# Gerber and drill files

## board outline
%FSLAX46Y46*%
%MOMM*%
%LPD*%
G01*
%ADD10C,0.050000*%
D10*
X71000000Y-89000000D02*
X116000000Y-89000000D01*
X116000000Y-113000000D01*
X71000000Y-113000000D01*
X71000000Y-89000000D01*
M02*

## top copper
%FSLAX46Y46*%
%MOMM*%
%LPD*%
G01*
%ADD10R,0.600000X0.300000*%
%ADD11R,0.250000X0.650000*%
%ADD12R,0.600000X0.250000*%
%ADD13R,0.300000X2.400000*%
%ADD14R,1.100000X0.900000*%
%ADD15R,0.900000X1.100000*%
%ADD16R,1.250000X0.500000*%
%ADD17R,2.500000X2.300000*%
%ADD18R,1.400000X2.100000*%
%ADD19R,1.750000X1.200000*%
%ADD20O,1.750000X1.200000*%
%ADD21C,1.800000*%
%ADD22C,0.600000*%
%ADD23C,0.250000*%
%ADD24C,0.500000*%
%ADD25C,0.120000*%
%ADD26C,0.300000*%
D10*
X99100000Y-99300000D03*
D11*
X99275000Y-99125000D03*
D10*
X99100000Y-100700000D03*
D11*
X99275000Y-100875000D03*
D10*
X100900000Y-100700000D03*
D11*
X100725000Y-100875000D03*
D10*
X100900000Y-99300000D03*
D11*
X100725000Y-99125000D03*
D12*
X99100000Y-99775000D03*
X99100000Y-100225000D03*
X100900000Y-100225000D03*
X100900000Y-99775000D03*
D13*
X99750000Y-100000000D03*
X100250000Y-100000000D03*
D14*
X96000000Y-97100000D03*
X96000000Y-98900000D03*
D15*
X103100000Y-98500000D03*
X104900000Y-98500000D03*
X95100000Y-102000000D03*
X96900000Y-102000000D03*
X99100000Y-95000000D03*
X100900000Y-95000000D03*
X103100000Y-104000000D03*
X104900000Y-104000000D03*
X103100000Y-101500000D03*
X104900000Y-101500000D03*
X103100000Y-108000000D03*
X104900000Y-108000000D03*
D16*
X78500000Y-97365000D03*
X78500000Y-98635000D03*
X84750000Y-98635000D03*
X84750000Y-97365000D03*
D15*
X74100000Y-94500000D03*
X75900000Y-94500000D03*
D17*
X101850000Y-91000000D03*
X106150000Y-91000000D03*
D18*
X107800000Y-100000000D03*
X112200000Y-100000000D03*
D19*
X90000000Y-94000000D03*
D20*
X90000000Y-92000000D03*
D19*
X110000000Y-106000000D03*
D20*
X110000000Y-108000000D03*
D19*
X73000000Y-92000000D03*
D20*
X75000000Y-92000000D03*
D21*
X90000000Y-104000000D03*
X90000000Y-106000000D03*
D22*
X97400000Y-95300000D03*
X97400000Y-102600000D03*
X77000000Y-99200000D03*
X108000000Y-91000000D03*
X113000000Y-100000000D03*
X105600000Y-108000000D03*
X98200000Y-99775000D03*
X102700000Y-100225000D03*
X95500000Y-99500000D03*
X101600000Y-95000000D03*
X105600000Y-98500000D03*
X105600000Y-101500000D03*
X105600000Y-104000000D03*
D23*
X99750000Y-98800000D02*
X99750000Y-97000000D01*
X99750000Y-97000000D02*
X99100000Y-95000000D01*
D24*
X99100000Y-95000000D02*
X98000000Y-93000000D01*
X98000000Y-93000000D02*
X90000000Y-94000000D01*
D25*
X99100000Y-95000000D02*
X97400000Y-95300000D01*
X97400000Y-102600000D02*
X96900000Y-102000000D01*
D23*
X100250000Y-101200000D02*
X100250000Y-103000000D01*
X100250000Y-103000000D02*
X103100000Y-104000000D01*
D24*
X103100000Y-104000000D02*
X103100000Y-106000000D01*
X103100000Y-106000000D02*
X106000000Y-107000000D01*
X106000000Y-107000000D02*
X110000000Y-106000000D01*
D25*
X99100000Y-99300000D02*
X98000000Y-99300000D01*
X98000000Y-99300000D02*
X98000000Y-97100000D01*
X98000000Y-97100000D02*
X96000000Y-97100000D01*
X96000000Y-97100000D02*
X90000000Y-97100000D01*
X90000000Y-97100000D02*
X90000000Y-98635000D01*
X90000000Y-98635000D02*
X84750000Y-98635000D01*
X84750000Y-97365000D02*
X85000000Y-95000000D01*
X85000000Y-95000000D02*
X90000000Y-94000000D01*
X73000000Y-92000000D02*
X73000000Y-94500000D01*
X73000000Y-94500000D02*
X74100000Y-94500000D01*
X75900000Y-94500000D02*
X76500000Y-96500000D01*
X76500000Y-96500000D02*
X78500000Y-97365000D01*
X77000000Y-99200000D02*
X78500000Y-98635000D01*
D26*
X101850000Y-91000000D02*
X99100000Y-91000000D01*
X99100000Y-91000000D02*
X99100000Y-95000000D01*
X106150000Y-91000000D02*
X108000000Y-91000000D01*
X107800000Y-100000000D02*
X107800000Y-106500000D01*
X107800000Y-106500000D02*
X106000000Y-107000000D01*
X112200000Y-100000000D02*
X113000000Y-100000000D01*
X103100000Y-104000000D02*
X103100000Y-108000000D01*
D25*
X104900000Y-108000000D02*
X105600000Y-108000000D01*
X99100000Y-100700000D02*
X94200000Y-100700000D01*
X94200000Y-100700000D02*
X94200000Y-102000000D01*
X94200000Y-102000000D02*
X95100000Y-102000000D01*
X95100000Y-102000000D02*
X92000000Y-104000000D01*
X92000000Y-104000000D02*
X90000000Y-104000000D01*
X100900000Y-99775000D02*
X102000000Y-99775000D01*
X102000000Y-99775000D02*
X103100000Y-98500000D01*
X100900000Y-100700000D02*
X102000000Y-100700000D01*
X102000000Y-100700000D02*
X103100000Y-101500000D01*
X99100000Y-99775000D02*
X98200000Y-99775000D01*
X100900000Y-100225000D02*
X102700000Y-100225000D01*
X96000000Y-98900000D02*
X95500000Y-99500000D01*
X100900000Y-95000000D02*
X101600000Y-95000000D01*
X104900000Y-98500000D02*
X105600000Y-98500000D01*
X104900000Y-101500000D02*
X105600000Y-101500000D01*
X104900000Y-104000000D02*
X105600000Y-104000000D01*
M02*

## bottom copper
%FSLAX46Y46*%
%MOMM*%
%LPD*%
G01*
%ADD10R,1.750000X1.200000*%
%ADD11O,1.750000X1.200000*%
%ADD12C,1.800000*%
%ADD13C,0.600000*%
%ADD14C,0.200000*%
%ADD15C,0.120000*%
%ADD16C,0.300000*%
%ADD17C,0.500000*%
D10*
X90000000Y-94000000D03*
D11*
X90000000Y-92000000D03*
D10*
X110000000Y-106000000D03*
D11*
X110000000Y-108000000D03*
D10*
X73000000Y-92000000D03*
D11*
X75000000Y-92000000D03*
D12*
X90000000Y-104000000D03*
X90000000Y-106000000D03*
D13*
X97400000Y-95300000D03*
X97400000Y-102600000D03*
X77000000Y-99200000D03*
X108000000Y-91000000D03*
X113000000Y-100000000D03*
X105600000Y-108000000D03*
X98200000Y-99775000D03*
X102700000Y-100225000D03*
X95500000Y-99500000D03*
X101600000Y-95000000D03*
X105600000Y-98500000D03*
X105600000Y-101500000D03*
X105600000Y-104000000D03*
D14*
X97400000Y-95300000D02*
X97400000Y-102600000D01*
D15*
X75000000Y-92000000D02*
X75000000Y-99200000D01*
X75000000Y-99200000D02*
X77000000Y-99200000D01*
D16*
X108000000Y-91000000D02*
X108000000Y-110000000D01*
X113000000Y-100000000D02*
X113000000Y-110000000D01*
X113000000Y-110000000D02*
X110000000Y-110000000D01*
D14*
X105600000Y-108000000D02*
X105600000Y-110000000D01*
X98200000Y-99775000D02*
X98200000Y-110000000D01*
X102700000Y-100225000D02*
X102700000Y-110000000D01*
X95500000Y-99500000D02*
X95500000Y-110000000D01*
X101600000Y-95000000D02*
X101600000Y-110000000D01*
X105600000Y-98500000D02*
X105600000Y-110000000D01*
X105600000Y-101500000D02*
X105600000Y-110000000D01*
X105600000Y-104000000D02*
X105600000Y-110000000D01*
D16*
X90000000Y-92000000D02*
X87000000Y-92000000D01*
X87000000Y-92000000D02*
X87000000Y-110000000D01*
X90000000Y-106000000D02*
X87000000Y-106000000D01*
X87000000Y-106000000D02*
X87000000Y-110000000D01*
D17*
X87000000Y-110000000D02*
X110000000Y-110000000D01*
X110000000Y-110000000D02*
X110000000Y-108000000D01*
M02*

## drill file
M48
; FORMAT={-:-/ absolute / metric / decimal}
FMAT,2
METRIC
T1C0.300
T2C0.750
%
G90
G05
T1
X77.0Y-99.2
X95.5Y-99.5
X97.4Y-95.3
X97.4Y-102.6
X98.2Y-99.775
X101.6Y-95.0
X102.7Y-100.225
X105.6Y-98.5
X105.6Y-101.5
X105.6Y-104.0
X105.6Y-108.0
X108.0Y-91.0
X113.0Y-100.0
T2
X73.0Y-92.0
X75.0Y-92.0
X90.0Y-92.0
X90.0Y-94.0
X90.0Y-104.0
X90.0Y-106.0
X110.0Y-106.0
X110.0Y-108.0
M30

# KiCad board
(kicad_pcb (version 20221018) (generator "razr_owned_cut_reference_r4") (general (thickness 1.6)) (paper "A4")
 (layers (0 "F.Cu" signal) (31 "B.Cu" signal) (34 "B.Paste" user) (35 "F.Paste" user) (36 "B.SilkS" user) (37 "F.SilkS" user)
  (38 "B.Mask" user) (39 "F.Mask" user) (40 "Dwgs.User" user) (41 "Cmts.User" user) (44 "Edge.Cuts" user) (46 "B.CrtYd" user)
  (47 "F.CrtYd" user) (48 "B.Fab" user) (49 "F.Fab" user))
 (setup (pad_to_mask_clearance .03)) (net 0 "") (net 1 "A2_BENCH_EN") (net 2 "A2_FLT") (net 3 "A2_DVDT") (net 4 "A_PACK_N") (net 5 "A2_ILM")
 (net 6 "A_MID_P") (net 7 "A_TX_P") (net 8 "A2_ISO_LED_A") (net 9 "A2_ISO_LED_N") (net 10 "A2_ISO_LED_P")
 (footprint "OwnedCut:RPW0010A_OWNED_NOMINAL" (layer "F.Cu") (at 100 100)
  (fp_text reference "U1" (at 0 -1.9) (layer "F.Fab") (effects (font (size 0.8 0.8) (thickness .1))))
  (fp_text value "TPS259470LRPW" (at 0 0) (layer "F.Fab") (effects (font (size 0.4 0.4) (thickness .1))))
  (pad "1" smd rect (at -0.9 -0.7) (size 0.6 0.3) (layers "F.Cu" "F.Paste" "F.Mask") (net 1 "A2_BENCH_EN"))
  (pad "1" smd rect (at -0.725 -0.875) (size 0.25 0.65) (layers "F.Cu" "F.Paste" "F.Mask") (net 1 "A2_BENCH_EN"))
  (pad "4" smd rect (at -0.9 0.7) (size 0.6 0.3) (layers "F.Cu" "F.Paste" "F.Mask") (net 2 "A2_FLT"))
  (pad "4" smd rect (at -0.725 0.875) (size 0.25 0.65) (layers "F.Cu" "F.Paste" "F.Mask") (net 2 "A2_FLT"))
  (pad "7" smd rect (at 0.9 0.7) (size 0.6 0.3) (layers "F.Cu" "F.Paste" "F.Mask") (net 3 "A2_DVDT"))
  (pad "7" smd rect (at 0.725 0.875) (size 0.25 0.65) (layers "F.Cu" "F.Paste" "F.Mask") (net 3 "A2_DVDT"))
  (pad "10" smd rect (at 0.9 -0.7) (size 0.6 0.3) (layers "F.Cu" "F.Paste" "F.Mask"))
  (pad "10" smd rect (at 0.725 -0.875) (size 0.25 0.65) (layers "F.Cu" "F.Paste" "F.Mask"))
  (pad "2" smd rect (at -0.9 -0.225) (size 0.6 0.25) (layers "F.Cu" "F.Paste" "F.Mask") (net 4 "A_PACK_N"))
  (pad "3" smd rect (at -0.9 0.225) (size 0.6 0.25) (layers "F.Cu" "F.Paste" "F.Mask"))
  (pad "8" smd rect (at 0.9 0.225) (size 0.6 0.25) (layers "F.Cu" "F.Paste" "F.Mask") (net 4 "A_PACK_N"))
  (pad "9" smd rect (at 0.9 -0.225) (size 0.6 0.25) (layers "F.Cu" "F.Paste" "F.Mask") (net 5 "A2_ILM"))
  (pad "5" smd rect (at -0.25 0) (size 0.3 2.4) (layers "F.Cu" "F.Paste" "F.Mask") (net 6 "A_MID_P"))
  (pad "6" smd rect (at 0.25 0) (size 0.3 2.4) (layers "F.Cu" "F.Paste" "F.Mask") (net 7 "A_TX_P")))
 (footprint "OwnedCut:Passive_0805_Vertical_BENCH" (layer "F.Cu") (at 96 98)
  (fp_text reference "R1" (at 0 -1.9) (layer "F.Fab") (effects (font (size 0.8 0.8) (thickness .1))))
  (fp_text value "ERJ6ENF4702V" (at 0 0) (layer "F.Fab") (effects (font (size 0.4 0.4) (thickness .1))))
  (pad "1" smd rect (at 0 -0.9) (size 1.1 0.9) (layers "F.Cu" "F.Paste" "F.Mask") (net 1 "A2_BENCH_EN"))
  (pad "2" smd rect (at 0 0.9) (size 1.1 0.9) (layers "F.Cu" "F.Paste" "F.Mask") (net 4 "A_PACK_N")))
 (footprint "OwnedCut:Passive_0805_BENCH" (layer "F.Cu") (at 104 98.5)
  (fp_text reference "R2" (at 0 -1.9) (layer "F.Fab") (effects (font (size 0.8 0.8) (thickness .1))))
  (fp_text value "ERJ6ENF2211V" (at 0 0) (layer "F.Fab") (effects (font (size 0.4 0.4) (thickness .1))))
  (pad "1" smd rect (at -0.9 0) (size 0.9 1.1) (layers "F.Cu" "F.Paste" "F.Mask") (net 5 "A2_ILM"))
  (pad "2" smd rect (at 0.9 0) (size 0.9 1.1) (layers "F.Cu" "F.Paste" "F.Mask") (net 4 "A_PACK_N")))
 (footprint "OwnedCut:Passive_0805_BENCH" (layer "F.Cu") (at 96 102)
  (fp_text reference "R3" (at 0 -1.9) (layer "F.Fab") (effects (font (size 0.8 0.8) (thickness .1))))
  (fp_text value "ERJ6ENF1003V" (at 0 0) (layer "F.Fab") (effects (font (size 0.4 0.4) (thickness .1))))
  (pad "1" smd rect (at -0.9 0) (size 0.9 1.1) (layers "F.Cu" "F.Paste" "F.Mask") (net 2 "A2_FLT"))
  (pad "2" smd rect (at 0.9 0) (size 0.9 1.1) (layers "F.Cu" "F.Paste" "F.Mask") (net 6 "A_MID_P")))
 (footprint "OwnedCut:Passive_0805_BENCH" (layer "F.Cu") (at 100 95)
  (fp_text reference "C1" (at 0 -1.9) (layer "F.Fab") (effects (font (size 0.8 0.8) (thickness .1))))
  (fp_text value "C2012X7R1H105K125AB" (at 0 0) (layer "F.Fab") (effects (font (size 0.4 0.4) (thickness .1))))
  (pad "1" smd rect (at -0.9 0) (size 0.9 1.1) (layers "F.Cu" "F.Paste" "F.Mask") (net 6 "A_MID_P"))
  (pad "2" smd rect (at 0.9 0) (size 0.9 1.1) (layers "F.Cu" "F.Paste" "F.Mask") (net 4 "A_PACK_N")))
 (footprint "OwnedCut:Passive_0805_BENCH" (layer "F.Cu") (at 104 104)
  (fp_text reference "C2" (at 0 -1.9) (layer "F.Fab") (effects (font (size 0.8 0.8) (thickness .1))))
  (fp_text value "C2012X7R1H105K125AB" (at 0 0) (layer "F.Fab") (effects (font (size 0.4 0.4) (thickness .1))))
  (pad "1" smd rect (at -0.9 0) (size 0.9 1.1) (layers "F.Cu" "F.Paste" "F.Mask") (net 7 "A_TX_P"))
  (pad "2" smd rect (at 0.9 0) (size 0.9 1.1) (layers "F.Cu" "F.Paste" "F.Mask") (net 4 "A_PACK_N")))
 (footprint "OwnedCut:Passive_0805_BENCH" (layer "F.Cu") (at 104 101.5)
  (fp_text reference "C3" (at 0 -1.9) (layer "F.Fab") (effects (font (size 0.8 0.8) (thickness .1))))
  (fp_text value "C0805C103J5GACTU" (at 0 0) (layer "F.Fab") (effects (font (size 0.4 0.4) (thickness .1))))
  (pad "1" smd rect (at -0.9 0) (size 0.9 1.1) (layers "F.Cu" "F.Paste" "F.Mask") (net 3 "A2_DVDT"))
  (pad "2" smd rect (at 0.9 0) (size 0.9 1.1) (layers "F.Cu" "F.Paste" "F.Mask") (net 4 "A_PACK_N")))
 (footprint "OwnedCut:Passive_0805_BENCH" (layer "F.Cu") (at 104 108)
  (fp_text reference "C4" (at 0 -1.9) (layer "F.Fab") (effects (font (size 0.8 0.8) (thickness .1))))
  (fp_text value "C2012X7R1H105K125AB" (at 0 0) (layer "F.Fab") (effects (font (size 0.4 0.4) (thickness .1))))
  (pad "1" smd rect (at -0.9 0) (size 0.9 1.1) (layers "F.Cu" "F.Paste" "F.Mask") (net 7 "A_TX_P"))
  (pad "2" smd rect (at 0.9 0) (size 0.9 1.1) (layers "F.Cu" "F.Paste" "F.Mask") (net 4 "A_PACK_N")))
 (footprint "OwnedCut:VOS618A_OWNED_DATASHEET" (layer "F.Cu") (at 81.625 98)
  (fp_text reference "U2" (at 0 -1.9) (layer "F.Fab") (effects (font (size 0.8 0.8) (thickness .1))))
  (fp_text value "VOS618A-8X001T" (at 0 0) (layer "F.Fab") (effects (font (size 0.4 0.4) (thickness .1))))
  (pad "1" smd rect (at -3.125 -0.635) (size 1.25 0.5) (layers "F.Cu" "F.Paste" "F.Mask") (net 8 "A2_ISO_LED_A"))
  (pad "2" smd rect (at -3.125 0.635) (size 1.25 0.5) (layers "F.Cu" "F.Paste" "F.Mask") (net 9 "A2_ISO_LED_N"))
  (pad "3" smd rect (at 3.125 0.635) (size 1.25 0.5) (layers "F.Cu" "F.Paste" "F.Mask") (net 1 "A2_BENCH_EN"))
  (pad "4" smd rect (at 3.125 -0.635) (size 1.25 0.5) (layers "F.Cu" "F.Paste" "F.Mask") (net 6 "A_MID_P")))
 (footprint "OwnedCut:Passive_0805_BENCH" (layer "F.Cu") (at 75 94.5)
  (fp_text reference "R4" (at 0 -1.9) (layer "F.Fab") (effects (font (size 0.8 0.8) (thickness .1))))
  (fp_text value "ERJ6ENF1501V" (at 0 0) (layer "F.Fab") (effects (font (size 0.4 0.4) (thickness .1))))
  (pad "1" smd rect (at -0.9 0) (size 0.9 1.1) (layers "F.Cu" "F.Paste" "F.Mask") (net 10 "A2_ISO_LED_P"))
  (pad "2" smd rect (at 0.9 0) (size 0.9 1.1) (layers "F.Cu" "F.Paste" "F.Mask") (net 8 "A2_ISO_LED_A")))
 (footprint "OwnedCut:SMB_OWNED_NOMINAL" (layer "F.Cu") (at 104 91)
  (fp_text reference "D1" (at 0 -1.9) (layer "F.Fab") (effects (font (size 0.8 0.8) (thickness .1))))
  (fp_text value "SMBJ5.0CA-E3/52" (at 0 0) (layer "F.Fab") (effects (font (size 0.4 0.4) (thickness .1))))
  (pad "1" smd rect (at -2.15 0) (size 2.5 2.3) (layers "F.Cu" "F.Paste" "F.Mask") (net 6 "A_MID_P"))
  (pad "2" smd rect (at 2.15 0) (size 2.5 2.3) (layers "F.Cu" "F.Paste" "F.Mask") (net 4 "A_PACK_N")))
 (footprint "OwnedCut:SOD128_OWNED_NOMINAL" (layer "F.Cu") (at 110 100)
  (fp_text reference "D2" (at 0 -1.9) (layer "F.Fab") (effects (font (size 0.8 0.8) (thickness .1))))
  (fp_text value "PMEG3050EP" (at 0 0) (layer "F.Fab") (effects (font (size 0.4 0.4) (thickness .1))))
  (pad "1" smd rect (at -2.2 0) (size 1.4 2.1) (layers "F.Cu" "F.Paste" "F.Mask") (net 7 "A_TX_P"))
  (pad "2" smd rect (at 2.2 0) (size 1.4 2.1) (layers "F.Cu" "F.Paste" "F.Mask") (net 4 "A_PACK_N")))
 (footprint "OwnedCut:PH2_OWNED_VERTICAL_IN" (layer "F.Cu") (at 90 94)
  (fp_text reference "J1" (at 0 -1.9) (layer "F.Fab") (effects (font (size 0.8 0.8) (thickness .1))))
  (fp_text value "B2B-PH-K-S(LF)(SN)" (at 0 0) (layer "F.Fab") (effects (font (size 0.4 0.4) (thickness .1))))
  (pad "1" thru_hole rect (at 0 0) (size 1.75 1.2) (drill .75) (layers "*.Cu" "*.Mask") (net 6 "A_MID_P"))
  (pad "2" thru_hole oval (at 0 -2) (size 1.75 1.2) (drill .75) (layers "*.Cu" "*.Mask") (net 4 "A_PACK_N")))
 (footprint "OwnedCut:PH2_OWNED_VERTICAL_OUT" (layer "F.Cu") (at 110 106)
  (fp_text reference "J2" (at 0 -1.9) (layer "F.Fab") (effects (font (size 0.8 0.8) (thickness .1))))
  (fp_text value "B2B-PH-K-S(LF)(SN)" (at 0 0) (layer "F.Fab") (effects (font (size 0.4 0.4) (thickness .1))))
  (pad "1" thru_hole rect (at 0 0) (size 1.75 1.2) (drill .75) (layers "*.Cu" "*.Mask") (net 7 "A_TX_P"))
  (pad "2" thru_hole oval (at 0 2) (size 1.75 1.2) (drill .75) (layers "*.Cu" "*.Mask") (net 4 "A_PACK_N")))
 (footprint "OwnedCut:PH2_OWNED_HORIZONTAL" (layer "F.Cu") (at 73 92)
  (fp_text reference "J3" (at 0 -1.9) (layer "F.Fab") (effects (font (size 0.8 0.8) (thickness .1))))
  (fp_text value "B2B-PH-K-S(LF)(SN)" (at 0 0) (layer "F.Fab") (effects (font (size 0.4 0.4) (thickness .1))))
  (pad "1" thru_hole rect (at 0 0) (size 1.75 1.2) (drill .75) (layers "*.Cu" "*.Mask") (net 10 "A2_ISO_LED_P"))
  (pad "2" thru_hole oval (at 2 0) (size 1.75 1.2) (drill .75) (layers "*.Cu" "*.Mask") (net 9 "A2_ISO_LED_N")))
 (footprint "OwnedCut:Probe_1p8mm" (layer "F.Cu") (at 90 104)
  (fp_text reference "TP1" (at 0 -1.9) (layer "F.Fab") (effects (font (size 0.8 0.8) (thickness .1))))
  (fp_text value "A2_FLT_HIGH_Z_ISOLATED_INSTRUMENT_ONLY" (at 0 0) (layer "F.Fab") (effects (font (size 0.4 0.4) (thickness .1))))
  (pad "1" thru_hole circle (at 0 0) (size 1.8 1.8) (drill .75) (layers "*.Cu" "*.Mask") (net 2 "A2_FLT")))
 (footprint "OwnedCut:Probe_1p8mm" (layer "F.Cu") (at 90 106)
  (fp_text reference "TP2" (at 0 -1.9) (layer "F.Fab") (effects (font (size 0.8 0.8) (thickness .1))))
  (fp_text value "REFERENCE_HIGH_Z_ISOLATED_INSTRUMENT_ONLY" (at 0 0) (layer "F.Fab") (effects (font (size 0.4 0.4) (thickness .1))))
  (pad "1" thru_hole circle (at 0 0) (size 1.8 1.8) (drill .75) (layers "*.Cu" "*.Mask") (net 4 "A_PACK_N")))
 (segment (start 99.75 98.8) (end 99.75 97) (width 0.25) (layer "F.Cu") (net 6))
 (segment (start 99.75 97) (end 99.1 95) (width 0.25) (layer "F.Cu") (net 6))
 (segment (start 99.1 95) (end 98 93) (width 0.5) (layer "F.Cu") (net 6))
 (segment (start 98 93) (end 90 94) (width 0.5) (layer "F.Cu") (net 6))
 (segment (start 99.1 95) (end 97.4 95.3) (width 0.12) (layer "F.Cu") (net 6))
 (via (at 97.4 95.3) (size .6) (drill .3) (layers "F.Cu" "B.Cu") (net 6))
 (segment (start 97.4 95.3) (end 97.4 102.6) (width 0.2) (layer "B.Cu") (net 6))
 (via (at 97.4 102.6) (size .6) (drill .3) (layers "F.Cu" "B.Cu") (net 6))
 (segment (start 97.4 102.6) (end 96.9 102) (width 0.12) (layer "F.Cu") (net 6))
 (segment (start 100.25 101.2) (end 100.25 103) (width 0.25) (layer "F.Cu") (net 7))
 (segment (start 100.25 103) (end 103.1 104) (width 0.25) (layer "F.Cu") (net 7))
 (segment (start 103.1 104) (end 103.1 106) (width 0.5) (layer "F.Cu") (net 7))
 (segment (start 103.1 106) (end 106 107) (width 0.5) (layer "F.Cu") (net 7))
 (segment (start 106 107) (end 110 106) (width 0.5) (layer "F.Cu") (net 7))
 (segment (start 99.1 99.3) (end 98 99.3) (width 0.12) (layer "F.Cu") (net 1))
 (segment (start 98 99.3) (end 98 97.1) (width 0.12) (layer "F.Cu") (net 1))
 (segment (start 98 97.1) (end 96 97.1) (width 0.12) (layer "F.Cu") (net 1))
 (segment (start 96 97.1) (end 90 97.1) (width 0.12) (layer "F.Cu") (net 1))
 (segment (start 90 97.1) (end 90 98.635) (width 0.12) (layer "F.Cu") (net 1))
 (segment (start 90 98.635) (end 84.75 98.635) (width 0.12) (layer "F.Cu") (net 1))
 (segment (start 84.75 97.365) (end 85 95) (width 0.12) (layer "F.Cu") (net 6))
 (segment (start 85 95) (end 90 94) (width 0.12) (layer "F.Cu") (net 6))
 (segment (start 73 92) (end 73 94.5) (width 0.12) (layer "F.Cu") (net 10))
 (segment (start 73 94.5) (end 74.1 94.5) (width 0.12) (layer "F.Cu") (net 10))
 (segment (start 75.9 94.5) (end 76.5 96.5) (width 0.12) (layer "F.Cu") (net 8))
 (segment (start 76.5 96.5) (end 78.5 97.365) (width 0.12) (layer "F.Cu") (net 8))
 (segment (start 75 92) (end 75 99.2) (width 0.12) (layer "B.Cu") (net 9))
 (segment (start 75 99.2) (end 77 99.2) (width 0.12) (layer "B.Cu") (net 9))
 (via (at 77 99.2) (size .6) (drill .3) (layers "F.Cu" "B.Cu") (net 9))
 (segment (start 77 99.2) (end 78.5 98.635) (width 0.12) (layer "F.Cu") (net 9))
 (segment (start 101.85 91) (end 99.1 91) (width 0.3) (layer "F.Cu") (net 6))
 (segment (start 99.1 91) (end 99.1 95) (width 0.3) (layer "F.Cu") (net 6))
 (segment (start 106.15 91) (end 108 91) (width 0.3) (layer "F.Cu") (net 4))
 (via (at 108 91) (size .6) (drill .3) (layers "F.Cu" "B.Cu") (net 4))
 (segment (start 108 91) (end 108 110) (width 0.3) (layer "B.Cu") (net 4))
 (segment (start 107.8 100) (end 107.8 106.5) (width 0.3) (layer "F.Cu") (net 7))
 (segment (start 107.8 106.5) (end 106 107) (width 0.3) (layer "F.Cu") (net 7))
 (segment (start 112.2 100) (end 113 100) (width 0.3) (layer "F.Cu") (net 4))
 (via (at 113 100) (size .6) (drill .3) (layers "F.Cu" "B.Cu") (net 4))
 (segment (start 113 100) (end 113 110) (width 0.3) (layer "B.Cu") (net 4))
 (segment (start 113 110) (end 110 110) (width 0.3) (layer "B.Cu") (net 4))
 (segment (start 103.1 104) (end 103.1 108) (width 0.3) (layer "F.Cu") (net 7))
 (segment (start 104.9 108) (end 105.6 108) (width 0.12) (layer "F.Cu") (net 4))
 (via (at 105.6 108) (size .6) (drill .3) (layers "F.Cu" "B.Cu") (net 4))
 (segment (start 105.6 108) (end 105.6 110) (width 0.2) (layer "B.Cu") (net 4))
 (segment (start 99.1 100.7) (end 94.2 100.7) (width 0.12) (layer "F.Cu") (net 2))
 (segment (start 94.2 100.7) (end 94.2 102) (width 0.12) (layer "F.Cu") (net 2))
 (segment (start 94.2 102) (end 95.1 102) (width 0.12) (layer "F.Cu") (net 2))
 (segment (start 95.1 102) (end 92 104) (width 0.12) (layer "F.Cu") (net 2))
 (segment (start 92 104) (end 90 104) (width 0.12) (layer "F.Cu") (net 2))
 (segment (start 100.9 99.775) (end 102 99.775) (width 0.12) (layer "F.Cu") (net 5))
 (segment (start 102 99.775) (end 103.1 98.5) (width 0.12) (layer "F.Cu") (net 5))
 (segment (start 100.9 100.7) (end 102 100.7) (width 0.12) (layer "F.Cu") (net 3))
 (segment (start 102 100.7) (end 103.1 101.5) (width 0.12) (layer "F.Cu") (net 3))
 (segment (start 99.1 99.775) (end 98.2 99.775) (width 0.12) (layer "F.Cu") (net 4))
 (via (at 98.2 99.775) (size .6) (drill .3) (layers "F.Cu" "B.Cu") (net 4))
 (segment (start 98.2 99.775) (end 98.2 110) (width 0.2) (layer "B.Cu") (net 4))
 (segment (start 100.9 100.225) (end 102.7 100.225) (width 0.12) (layer "F.Cu") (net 4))
 (via (at 102.7 100.225) (size .6) (drill .3) (layers "F.Cu" "B.Cu") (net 4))
 (segment (start 102.7 100.225) (end 102.7 110) (width 0.2) (layer "B.Cu") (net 4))
 (segment (start 96 98.9) (end 95.5 99.5) (width 0.12) (layer "F.Cu") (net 4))
 (via (at 95.5 99.5) (size .6) (drill .3) (layers "F.Cu" "B.Cu") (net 4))
 (segment (start 95.5 99.5) (end 95.5 110) (width 0.2) (layer "B.Cu") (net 4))
 (segment (start 100.9 95) (end 101.6 95) (width 0.12) (layer "F.Cu") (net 4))
 (via (at 101.6 95) (size .6) (drill .3) (layers "F.Cu" "B.Cu") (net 4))
 (segment (start 101.6 95) (end 101.6 110) (width 0.2) (layer "B.Cu") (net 4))
 (segment (start 104.9 98.5) (end 105.6 98.5) (width 0.12) (layer "F.Cu") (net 4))
 (via (at 105.6 98.5) (size .6) (drill .3) (layers "F.Cu" "B.Cu") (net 4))
 (segment (start 105.6 98.5) (end 105.6 110) (width 0.2) (layer "B.Cu") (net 4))
 (segment (start 104.9 101.5) (end 105.6 101.5) (width 0.12) (layer "F.Cu") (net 4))
 (via (at 105.6 101.5) (size .6) (drill .3) (layers "F.Cu" "B.Cu") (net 4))
 (segment (start 105.6 101.5) (end 105.6 110) (width 0.2) (layer "B.Cu") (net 4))
 (segment (start 104.9 104) (end 105.6 104) (width 0.12) (layer "F.Cu") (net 4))
 (via (at 105.6 104) (size .6) (drill .3) (layers "F.Cu" "B.Cu") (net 4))
 (segment (start 105.6 104) (end 105.6 110) (width 0.2) (layer "B.Cu") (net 4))
 (segment (start 90 92) (end 87 92) (width 0.3) (layer "B.Cu") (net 4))
 (segment (start 87 92) (end 87 110) (width 0.3) (layer "B.Cu") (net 4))
 (segment (start 90 106) (end 87 106) (width 0.3) (layer "B.Cu") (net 4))
 (segment (start 87 106) (end 87 110) (width 0.3) (layer "B.Cu") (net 4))
 (segment (start 87 110) (end 110 110) (width 0.5) (layer "B.Cu") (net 4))
 (segment (start 110 110) (end 110 108) (width 0.5) (layer "B.Cu") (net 4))
 (gr_rect (start 71 89) (end 116 113) (stroke (width .05) (type default)) (fill none) (layer "Edge.Cuts")))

